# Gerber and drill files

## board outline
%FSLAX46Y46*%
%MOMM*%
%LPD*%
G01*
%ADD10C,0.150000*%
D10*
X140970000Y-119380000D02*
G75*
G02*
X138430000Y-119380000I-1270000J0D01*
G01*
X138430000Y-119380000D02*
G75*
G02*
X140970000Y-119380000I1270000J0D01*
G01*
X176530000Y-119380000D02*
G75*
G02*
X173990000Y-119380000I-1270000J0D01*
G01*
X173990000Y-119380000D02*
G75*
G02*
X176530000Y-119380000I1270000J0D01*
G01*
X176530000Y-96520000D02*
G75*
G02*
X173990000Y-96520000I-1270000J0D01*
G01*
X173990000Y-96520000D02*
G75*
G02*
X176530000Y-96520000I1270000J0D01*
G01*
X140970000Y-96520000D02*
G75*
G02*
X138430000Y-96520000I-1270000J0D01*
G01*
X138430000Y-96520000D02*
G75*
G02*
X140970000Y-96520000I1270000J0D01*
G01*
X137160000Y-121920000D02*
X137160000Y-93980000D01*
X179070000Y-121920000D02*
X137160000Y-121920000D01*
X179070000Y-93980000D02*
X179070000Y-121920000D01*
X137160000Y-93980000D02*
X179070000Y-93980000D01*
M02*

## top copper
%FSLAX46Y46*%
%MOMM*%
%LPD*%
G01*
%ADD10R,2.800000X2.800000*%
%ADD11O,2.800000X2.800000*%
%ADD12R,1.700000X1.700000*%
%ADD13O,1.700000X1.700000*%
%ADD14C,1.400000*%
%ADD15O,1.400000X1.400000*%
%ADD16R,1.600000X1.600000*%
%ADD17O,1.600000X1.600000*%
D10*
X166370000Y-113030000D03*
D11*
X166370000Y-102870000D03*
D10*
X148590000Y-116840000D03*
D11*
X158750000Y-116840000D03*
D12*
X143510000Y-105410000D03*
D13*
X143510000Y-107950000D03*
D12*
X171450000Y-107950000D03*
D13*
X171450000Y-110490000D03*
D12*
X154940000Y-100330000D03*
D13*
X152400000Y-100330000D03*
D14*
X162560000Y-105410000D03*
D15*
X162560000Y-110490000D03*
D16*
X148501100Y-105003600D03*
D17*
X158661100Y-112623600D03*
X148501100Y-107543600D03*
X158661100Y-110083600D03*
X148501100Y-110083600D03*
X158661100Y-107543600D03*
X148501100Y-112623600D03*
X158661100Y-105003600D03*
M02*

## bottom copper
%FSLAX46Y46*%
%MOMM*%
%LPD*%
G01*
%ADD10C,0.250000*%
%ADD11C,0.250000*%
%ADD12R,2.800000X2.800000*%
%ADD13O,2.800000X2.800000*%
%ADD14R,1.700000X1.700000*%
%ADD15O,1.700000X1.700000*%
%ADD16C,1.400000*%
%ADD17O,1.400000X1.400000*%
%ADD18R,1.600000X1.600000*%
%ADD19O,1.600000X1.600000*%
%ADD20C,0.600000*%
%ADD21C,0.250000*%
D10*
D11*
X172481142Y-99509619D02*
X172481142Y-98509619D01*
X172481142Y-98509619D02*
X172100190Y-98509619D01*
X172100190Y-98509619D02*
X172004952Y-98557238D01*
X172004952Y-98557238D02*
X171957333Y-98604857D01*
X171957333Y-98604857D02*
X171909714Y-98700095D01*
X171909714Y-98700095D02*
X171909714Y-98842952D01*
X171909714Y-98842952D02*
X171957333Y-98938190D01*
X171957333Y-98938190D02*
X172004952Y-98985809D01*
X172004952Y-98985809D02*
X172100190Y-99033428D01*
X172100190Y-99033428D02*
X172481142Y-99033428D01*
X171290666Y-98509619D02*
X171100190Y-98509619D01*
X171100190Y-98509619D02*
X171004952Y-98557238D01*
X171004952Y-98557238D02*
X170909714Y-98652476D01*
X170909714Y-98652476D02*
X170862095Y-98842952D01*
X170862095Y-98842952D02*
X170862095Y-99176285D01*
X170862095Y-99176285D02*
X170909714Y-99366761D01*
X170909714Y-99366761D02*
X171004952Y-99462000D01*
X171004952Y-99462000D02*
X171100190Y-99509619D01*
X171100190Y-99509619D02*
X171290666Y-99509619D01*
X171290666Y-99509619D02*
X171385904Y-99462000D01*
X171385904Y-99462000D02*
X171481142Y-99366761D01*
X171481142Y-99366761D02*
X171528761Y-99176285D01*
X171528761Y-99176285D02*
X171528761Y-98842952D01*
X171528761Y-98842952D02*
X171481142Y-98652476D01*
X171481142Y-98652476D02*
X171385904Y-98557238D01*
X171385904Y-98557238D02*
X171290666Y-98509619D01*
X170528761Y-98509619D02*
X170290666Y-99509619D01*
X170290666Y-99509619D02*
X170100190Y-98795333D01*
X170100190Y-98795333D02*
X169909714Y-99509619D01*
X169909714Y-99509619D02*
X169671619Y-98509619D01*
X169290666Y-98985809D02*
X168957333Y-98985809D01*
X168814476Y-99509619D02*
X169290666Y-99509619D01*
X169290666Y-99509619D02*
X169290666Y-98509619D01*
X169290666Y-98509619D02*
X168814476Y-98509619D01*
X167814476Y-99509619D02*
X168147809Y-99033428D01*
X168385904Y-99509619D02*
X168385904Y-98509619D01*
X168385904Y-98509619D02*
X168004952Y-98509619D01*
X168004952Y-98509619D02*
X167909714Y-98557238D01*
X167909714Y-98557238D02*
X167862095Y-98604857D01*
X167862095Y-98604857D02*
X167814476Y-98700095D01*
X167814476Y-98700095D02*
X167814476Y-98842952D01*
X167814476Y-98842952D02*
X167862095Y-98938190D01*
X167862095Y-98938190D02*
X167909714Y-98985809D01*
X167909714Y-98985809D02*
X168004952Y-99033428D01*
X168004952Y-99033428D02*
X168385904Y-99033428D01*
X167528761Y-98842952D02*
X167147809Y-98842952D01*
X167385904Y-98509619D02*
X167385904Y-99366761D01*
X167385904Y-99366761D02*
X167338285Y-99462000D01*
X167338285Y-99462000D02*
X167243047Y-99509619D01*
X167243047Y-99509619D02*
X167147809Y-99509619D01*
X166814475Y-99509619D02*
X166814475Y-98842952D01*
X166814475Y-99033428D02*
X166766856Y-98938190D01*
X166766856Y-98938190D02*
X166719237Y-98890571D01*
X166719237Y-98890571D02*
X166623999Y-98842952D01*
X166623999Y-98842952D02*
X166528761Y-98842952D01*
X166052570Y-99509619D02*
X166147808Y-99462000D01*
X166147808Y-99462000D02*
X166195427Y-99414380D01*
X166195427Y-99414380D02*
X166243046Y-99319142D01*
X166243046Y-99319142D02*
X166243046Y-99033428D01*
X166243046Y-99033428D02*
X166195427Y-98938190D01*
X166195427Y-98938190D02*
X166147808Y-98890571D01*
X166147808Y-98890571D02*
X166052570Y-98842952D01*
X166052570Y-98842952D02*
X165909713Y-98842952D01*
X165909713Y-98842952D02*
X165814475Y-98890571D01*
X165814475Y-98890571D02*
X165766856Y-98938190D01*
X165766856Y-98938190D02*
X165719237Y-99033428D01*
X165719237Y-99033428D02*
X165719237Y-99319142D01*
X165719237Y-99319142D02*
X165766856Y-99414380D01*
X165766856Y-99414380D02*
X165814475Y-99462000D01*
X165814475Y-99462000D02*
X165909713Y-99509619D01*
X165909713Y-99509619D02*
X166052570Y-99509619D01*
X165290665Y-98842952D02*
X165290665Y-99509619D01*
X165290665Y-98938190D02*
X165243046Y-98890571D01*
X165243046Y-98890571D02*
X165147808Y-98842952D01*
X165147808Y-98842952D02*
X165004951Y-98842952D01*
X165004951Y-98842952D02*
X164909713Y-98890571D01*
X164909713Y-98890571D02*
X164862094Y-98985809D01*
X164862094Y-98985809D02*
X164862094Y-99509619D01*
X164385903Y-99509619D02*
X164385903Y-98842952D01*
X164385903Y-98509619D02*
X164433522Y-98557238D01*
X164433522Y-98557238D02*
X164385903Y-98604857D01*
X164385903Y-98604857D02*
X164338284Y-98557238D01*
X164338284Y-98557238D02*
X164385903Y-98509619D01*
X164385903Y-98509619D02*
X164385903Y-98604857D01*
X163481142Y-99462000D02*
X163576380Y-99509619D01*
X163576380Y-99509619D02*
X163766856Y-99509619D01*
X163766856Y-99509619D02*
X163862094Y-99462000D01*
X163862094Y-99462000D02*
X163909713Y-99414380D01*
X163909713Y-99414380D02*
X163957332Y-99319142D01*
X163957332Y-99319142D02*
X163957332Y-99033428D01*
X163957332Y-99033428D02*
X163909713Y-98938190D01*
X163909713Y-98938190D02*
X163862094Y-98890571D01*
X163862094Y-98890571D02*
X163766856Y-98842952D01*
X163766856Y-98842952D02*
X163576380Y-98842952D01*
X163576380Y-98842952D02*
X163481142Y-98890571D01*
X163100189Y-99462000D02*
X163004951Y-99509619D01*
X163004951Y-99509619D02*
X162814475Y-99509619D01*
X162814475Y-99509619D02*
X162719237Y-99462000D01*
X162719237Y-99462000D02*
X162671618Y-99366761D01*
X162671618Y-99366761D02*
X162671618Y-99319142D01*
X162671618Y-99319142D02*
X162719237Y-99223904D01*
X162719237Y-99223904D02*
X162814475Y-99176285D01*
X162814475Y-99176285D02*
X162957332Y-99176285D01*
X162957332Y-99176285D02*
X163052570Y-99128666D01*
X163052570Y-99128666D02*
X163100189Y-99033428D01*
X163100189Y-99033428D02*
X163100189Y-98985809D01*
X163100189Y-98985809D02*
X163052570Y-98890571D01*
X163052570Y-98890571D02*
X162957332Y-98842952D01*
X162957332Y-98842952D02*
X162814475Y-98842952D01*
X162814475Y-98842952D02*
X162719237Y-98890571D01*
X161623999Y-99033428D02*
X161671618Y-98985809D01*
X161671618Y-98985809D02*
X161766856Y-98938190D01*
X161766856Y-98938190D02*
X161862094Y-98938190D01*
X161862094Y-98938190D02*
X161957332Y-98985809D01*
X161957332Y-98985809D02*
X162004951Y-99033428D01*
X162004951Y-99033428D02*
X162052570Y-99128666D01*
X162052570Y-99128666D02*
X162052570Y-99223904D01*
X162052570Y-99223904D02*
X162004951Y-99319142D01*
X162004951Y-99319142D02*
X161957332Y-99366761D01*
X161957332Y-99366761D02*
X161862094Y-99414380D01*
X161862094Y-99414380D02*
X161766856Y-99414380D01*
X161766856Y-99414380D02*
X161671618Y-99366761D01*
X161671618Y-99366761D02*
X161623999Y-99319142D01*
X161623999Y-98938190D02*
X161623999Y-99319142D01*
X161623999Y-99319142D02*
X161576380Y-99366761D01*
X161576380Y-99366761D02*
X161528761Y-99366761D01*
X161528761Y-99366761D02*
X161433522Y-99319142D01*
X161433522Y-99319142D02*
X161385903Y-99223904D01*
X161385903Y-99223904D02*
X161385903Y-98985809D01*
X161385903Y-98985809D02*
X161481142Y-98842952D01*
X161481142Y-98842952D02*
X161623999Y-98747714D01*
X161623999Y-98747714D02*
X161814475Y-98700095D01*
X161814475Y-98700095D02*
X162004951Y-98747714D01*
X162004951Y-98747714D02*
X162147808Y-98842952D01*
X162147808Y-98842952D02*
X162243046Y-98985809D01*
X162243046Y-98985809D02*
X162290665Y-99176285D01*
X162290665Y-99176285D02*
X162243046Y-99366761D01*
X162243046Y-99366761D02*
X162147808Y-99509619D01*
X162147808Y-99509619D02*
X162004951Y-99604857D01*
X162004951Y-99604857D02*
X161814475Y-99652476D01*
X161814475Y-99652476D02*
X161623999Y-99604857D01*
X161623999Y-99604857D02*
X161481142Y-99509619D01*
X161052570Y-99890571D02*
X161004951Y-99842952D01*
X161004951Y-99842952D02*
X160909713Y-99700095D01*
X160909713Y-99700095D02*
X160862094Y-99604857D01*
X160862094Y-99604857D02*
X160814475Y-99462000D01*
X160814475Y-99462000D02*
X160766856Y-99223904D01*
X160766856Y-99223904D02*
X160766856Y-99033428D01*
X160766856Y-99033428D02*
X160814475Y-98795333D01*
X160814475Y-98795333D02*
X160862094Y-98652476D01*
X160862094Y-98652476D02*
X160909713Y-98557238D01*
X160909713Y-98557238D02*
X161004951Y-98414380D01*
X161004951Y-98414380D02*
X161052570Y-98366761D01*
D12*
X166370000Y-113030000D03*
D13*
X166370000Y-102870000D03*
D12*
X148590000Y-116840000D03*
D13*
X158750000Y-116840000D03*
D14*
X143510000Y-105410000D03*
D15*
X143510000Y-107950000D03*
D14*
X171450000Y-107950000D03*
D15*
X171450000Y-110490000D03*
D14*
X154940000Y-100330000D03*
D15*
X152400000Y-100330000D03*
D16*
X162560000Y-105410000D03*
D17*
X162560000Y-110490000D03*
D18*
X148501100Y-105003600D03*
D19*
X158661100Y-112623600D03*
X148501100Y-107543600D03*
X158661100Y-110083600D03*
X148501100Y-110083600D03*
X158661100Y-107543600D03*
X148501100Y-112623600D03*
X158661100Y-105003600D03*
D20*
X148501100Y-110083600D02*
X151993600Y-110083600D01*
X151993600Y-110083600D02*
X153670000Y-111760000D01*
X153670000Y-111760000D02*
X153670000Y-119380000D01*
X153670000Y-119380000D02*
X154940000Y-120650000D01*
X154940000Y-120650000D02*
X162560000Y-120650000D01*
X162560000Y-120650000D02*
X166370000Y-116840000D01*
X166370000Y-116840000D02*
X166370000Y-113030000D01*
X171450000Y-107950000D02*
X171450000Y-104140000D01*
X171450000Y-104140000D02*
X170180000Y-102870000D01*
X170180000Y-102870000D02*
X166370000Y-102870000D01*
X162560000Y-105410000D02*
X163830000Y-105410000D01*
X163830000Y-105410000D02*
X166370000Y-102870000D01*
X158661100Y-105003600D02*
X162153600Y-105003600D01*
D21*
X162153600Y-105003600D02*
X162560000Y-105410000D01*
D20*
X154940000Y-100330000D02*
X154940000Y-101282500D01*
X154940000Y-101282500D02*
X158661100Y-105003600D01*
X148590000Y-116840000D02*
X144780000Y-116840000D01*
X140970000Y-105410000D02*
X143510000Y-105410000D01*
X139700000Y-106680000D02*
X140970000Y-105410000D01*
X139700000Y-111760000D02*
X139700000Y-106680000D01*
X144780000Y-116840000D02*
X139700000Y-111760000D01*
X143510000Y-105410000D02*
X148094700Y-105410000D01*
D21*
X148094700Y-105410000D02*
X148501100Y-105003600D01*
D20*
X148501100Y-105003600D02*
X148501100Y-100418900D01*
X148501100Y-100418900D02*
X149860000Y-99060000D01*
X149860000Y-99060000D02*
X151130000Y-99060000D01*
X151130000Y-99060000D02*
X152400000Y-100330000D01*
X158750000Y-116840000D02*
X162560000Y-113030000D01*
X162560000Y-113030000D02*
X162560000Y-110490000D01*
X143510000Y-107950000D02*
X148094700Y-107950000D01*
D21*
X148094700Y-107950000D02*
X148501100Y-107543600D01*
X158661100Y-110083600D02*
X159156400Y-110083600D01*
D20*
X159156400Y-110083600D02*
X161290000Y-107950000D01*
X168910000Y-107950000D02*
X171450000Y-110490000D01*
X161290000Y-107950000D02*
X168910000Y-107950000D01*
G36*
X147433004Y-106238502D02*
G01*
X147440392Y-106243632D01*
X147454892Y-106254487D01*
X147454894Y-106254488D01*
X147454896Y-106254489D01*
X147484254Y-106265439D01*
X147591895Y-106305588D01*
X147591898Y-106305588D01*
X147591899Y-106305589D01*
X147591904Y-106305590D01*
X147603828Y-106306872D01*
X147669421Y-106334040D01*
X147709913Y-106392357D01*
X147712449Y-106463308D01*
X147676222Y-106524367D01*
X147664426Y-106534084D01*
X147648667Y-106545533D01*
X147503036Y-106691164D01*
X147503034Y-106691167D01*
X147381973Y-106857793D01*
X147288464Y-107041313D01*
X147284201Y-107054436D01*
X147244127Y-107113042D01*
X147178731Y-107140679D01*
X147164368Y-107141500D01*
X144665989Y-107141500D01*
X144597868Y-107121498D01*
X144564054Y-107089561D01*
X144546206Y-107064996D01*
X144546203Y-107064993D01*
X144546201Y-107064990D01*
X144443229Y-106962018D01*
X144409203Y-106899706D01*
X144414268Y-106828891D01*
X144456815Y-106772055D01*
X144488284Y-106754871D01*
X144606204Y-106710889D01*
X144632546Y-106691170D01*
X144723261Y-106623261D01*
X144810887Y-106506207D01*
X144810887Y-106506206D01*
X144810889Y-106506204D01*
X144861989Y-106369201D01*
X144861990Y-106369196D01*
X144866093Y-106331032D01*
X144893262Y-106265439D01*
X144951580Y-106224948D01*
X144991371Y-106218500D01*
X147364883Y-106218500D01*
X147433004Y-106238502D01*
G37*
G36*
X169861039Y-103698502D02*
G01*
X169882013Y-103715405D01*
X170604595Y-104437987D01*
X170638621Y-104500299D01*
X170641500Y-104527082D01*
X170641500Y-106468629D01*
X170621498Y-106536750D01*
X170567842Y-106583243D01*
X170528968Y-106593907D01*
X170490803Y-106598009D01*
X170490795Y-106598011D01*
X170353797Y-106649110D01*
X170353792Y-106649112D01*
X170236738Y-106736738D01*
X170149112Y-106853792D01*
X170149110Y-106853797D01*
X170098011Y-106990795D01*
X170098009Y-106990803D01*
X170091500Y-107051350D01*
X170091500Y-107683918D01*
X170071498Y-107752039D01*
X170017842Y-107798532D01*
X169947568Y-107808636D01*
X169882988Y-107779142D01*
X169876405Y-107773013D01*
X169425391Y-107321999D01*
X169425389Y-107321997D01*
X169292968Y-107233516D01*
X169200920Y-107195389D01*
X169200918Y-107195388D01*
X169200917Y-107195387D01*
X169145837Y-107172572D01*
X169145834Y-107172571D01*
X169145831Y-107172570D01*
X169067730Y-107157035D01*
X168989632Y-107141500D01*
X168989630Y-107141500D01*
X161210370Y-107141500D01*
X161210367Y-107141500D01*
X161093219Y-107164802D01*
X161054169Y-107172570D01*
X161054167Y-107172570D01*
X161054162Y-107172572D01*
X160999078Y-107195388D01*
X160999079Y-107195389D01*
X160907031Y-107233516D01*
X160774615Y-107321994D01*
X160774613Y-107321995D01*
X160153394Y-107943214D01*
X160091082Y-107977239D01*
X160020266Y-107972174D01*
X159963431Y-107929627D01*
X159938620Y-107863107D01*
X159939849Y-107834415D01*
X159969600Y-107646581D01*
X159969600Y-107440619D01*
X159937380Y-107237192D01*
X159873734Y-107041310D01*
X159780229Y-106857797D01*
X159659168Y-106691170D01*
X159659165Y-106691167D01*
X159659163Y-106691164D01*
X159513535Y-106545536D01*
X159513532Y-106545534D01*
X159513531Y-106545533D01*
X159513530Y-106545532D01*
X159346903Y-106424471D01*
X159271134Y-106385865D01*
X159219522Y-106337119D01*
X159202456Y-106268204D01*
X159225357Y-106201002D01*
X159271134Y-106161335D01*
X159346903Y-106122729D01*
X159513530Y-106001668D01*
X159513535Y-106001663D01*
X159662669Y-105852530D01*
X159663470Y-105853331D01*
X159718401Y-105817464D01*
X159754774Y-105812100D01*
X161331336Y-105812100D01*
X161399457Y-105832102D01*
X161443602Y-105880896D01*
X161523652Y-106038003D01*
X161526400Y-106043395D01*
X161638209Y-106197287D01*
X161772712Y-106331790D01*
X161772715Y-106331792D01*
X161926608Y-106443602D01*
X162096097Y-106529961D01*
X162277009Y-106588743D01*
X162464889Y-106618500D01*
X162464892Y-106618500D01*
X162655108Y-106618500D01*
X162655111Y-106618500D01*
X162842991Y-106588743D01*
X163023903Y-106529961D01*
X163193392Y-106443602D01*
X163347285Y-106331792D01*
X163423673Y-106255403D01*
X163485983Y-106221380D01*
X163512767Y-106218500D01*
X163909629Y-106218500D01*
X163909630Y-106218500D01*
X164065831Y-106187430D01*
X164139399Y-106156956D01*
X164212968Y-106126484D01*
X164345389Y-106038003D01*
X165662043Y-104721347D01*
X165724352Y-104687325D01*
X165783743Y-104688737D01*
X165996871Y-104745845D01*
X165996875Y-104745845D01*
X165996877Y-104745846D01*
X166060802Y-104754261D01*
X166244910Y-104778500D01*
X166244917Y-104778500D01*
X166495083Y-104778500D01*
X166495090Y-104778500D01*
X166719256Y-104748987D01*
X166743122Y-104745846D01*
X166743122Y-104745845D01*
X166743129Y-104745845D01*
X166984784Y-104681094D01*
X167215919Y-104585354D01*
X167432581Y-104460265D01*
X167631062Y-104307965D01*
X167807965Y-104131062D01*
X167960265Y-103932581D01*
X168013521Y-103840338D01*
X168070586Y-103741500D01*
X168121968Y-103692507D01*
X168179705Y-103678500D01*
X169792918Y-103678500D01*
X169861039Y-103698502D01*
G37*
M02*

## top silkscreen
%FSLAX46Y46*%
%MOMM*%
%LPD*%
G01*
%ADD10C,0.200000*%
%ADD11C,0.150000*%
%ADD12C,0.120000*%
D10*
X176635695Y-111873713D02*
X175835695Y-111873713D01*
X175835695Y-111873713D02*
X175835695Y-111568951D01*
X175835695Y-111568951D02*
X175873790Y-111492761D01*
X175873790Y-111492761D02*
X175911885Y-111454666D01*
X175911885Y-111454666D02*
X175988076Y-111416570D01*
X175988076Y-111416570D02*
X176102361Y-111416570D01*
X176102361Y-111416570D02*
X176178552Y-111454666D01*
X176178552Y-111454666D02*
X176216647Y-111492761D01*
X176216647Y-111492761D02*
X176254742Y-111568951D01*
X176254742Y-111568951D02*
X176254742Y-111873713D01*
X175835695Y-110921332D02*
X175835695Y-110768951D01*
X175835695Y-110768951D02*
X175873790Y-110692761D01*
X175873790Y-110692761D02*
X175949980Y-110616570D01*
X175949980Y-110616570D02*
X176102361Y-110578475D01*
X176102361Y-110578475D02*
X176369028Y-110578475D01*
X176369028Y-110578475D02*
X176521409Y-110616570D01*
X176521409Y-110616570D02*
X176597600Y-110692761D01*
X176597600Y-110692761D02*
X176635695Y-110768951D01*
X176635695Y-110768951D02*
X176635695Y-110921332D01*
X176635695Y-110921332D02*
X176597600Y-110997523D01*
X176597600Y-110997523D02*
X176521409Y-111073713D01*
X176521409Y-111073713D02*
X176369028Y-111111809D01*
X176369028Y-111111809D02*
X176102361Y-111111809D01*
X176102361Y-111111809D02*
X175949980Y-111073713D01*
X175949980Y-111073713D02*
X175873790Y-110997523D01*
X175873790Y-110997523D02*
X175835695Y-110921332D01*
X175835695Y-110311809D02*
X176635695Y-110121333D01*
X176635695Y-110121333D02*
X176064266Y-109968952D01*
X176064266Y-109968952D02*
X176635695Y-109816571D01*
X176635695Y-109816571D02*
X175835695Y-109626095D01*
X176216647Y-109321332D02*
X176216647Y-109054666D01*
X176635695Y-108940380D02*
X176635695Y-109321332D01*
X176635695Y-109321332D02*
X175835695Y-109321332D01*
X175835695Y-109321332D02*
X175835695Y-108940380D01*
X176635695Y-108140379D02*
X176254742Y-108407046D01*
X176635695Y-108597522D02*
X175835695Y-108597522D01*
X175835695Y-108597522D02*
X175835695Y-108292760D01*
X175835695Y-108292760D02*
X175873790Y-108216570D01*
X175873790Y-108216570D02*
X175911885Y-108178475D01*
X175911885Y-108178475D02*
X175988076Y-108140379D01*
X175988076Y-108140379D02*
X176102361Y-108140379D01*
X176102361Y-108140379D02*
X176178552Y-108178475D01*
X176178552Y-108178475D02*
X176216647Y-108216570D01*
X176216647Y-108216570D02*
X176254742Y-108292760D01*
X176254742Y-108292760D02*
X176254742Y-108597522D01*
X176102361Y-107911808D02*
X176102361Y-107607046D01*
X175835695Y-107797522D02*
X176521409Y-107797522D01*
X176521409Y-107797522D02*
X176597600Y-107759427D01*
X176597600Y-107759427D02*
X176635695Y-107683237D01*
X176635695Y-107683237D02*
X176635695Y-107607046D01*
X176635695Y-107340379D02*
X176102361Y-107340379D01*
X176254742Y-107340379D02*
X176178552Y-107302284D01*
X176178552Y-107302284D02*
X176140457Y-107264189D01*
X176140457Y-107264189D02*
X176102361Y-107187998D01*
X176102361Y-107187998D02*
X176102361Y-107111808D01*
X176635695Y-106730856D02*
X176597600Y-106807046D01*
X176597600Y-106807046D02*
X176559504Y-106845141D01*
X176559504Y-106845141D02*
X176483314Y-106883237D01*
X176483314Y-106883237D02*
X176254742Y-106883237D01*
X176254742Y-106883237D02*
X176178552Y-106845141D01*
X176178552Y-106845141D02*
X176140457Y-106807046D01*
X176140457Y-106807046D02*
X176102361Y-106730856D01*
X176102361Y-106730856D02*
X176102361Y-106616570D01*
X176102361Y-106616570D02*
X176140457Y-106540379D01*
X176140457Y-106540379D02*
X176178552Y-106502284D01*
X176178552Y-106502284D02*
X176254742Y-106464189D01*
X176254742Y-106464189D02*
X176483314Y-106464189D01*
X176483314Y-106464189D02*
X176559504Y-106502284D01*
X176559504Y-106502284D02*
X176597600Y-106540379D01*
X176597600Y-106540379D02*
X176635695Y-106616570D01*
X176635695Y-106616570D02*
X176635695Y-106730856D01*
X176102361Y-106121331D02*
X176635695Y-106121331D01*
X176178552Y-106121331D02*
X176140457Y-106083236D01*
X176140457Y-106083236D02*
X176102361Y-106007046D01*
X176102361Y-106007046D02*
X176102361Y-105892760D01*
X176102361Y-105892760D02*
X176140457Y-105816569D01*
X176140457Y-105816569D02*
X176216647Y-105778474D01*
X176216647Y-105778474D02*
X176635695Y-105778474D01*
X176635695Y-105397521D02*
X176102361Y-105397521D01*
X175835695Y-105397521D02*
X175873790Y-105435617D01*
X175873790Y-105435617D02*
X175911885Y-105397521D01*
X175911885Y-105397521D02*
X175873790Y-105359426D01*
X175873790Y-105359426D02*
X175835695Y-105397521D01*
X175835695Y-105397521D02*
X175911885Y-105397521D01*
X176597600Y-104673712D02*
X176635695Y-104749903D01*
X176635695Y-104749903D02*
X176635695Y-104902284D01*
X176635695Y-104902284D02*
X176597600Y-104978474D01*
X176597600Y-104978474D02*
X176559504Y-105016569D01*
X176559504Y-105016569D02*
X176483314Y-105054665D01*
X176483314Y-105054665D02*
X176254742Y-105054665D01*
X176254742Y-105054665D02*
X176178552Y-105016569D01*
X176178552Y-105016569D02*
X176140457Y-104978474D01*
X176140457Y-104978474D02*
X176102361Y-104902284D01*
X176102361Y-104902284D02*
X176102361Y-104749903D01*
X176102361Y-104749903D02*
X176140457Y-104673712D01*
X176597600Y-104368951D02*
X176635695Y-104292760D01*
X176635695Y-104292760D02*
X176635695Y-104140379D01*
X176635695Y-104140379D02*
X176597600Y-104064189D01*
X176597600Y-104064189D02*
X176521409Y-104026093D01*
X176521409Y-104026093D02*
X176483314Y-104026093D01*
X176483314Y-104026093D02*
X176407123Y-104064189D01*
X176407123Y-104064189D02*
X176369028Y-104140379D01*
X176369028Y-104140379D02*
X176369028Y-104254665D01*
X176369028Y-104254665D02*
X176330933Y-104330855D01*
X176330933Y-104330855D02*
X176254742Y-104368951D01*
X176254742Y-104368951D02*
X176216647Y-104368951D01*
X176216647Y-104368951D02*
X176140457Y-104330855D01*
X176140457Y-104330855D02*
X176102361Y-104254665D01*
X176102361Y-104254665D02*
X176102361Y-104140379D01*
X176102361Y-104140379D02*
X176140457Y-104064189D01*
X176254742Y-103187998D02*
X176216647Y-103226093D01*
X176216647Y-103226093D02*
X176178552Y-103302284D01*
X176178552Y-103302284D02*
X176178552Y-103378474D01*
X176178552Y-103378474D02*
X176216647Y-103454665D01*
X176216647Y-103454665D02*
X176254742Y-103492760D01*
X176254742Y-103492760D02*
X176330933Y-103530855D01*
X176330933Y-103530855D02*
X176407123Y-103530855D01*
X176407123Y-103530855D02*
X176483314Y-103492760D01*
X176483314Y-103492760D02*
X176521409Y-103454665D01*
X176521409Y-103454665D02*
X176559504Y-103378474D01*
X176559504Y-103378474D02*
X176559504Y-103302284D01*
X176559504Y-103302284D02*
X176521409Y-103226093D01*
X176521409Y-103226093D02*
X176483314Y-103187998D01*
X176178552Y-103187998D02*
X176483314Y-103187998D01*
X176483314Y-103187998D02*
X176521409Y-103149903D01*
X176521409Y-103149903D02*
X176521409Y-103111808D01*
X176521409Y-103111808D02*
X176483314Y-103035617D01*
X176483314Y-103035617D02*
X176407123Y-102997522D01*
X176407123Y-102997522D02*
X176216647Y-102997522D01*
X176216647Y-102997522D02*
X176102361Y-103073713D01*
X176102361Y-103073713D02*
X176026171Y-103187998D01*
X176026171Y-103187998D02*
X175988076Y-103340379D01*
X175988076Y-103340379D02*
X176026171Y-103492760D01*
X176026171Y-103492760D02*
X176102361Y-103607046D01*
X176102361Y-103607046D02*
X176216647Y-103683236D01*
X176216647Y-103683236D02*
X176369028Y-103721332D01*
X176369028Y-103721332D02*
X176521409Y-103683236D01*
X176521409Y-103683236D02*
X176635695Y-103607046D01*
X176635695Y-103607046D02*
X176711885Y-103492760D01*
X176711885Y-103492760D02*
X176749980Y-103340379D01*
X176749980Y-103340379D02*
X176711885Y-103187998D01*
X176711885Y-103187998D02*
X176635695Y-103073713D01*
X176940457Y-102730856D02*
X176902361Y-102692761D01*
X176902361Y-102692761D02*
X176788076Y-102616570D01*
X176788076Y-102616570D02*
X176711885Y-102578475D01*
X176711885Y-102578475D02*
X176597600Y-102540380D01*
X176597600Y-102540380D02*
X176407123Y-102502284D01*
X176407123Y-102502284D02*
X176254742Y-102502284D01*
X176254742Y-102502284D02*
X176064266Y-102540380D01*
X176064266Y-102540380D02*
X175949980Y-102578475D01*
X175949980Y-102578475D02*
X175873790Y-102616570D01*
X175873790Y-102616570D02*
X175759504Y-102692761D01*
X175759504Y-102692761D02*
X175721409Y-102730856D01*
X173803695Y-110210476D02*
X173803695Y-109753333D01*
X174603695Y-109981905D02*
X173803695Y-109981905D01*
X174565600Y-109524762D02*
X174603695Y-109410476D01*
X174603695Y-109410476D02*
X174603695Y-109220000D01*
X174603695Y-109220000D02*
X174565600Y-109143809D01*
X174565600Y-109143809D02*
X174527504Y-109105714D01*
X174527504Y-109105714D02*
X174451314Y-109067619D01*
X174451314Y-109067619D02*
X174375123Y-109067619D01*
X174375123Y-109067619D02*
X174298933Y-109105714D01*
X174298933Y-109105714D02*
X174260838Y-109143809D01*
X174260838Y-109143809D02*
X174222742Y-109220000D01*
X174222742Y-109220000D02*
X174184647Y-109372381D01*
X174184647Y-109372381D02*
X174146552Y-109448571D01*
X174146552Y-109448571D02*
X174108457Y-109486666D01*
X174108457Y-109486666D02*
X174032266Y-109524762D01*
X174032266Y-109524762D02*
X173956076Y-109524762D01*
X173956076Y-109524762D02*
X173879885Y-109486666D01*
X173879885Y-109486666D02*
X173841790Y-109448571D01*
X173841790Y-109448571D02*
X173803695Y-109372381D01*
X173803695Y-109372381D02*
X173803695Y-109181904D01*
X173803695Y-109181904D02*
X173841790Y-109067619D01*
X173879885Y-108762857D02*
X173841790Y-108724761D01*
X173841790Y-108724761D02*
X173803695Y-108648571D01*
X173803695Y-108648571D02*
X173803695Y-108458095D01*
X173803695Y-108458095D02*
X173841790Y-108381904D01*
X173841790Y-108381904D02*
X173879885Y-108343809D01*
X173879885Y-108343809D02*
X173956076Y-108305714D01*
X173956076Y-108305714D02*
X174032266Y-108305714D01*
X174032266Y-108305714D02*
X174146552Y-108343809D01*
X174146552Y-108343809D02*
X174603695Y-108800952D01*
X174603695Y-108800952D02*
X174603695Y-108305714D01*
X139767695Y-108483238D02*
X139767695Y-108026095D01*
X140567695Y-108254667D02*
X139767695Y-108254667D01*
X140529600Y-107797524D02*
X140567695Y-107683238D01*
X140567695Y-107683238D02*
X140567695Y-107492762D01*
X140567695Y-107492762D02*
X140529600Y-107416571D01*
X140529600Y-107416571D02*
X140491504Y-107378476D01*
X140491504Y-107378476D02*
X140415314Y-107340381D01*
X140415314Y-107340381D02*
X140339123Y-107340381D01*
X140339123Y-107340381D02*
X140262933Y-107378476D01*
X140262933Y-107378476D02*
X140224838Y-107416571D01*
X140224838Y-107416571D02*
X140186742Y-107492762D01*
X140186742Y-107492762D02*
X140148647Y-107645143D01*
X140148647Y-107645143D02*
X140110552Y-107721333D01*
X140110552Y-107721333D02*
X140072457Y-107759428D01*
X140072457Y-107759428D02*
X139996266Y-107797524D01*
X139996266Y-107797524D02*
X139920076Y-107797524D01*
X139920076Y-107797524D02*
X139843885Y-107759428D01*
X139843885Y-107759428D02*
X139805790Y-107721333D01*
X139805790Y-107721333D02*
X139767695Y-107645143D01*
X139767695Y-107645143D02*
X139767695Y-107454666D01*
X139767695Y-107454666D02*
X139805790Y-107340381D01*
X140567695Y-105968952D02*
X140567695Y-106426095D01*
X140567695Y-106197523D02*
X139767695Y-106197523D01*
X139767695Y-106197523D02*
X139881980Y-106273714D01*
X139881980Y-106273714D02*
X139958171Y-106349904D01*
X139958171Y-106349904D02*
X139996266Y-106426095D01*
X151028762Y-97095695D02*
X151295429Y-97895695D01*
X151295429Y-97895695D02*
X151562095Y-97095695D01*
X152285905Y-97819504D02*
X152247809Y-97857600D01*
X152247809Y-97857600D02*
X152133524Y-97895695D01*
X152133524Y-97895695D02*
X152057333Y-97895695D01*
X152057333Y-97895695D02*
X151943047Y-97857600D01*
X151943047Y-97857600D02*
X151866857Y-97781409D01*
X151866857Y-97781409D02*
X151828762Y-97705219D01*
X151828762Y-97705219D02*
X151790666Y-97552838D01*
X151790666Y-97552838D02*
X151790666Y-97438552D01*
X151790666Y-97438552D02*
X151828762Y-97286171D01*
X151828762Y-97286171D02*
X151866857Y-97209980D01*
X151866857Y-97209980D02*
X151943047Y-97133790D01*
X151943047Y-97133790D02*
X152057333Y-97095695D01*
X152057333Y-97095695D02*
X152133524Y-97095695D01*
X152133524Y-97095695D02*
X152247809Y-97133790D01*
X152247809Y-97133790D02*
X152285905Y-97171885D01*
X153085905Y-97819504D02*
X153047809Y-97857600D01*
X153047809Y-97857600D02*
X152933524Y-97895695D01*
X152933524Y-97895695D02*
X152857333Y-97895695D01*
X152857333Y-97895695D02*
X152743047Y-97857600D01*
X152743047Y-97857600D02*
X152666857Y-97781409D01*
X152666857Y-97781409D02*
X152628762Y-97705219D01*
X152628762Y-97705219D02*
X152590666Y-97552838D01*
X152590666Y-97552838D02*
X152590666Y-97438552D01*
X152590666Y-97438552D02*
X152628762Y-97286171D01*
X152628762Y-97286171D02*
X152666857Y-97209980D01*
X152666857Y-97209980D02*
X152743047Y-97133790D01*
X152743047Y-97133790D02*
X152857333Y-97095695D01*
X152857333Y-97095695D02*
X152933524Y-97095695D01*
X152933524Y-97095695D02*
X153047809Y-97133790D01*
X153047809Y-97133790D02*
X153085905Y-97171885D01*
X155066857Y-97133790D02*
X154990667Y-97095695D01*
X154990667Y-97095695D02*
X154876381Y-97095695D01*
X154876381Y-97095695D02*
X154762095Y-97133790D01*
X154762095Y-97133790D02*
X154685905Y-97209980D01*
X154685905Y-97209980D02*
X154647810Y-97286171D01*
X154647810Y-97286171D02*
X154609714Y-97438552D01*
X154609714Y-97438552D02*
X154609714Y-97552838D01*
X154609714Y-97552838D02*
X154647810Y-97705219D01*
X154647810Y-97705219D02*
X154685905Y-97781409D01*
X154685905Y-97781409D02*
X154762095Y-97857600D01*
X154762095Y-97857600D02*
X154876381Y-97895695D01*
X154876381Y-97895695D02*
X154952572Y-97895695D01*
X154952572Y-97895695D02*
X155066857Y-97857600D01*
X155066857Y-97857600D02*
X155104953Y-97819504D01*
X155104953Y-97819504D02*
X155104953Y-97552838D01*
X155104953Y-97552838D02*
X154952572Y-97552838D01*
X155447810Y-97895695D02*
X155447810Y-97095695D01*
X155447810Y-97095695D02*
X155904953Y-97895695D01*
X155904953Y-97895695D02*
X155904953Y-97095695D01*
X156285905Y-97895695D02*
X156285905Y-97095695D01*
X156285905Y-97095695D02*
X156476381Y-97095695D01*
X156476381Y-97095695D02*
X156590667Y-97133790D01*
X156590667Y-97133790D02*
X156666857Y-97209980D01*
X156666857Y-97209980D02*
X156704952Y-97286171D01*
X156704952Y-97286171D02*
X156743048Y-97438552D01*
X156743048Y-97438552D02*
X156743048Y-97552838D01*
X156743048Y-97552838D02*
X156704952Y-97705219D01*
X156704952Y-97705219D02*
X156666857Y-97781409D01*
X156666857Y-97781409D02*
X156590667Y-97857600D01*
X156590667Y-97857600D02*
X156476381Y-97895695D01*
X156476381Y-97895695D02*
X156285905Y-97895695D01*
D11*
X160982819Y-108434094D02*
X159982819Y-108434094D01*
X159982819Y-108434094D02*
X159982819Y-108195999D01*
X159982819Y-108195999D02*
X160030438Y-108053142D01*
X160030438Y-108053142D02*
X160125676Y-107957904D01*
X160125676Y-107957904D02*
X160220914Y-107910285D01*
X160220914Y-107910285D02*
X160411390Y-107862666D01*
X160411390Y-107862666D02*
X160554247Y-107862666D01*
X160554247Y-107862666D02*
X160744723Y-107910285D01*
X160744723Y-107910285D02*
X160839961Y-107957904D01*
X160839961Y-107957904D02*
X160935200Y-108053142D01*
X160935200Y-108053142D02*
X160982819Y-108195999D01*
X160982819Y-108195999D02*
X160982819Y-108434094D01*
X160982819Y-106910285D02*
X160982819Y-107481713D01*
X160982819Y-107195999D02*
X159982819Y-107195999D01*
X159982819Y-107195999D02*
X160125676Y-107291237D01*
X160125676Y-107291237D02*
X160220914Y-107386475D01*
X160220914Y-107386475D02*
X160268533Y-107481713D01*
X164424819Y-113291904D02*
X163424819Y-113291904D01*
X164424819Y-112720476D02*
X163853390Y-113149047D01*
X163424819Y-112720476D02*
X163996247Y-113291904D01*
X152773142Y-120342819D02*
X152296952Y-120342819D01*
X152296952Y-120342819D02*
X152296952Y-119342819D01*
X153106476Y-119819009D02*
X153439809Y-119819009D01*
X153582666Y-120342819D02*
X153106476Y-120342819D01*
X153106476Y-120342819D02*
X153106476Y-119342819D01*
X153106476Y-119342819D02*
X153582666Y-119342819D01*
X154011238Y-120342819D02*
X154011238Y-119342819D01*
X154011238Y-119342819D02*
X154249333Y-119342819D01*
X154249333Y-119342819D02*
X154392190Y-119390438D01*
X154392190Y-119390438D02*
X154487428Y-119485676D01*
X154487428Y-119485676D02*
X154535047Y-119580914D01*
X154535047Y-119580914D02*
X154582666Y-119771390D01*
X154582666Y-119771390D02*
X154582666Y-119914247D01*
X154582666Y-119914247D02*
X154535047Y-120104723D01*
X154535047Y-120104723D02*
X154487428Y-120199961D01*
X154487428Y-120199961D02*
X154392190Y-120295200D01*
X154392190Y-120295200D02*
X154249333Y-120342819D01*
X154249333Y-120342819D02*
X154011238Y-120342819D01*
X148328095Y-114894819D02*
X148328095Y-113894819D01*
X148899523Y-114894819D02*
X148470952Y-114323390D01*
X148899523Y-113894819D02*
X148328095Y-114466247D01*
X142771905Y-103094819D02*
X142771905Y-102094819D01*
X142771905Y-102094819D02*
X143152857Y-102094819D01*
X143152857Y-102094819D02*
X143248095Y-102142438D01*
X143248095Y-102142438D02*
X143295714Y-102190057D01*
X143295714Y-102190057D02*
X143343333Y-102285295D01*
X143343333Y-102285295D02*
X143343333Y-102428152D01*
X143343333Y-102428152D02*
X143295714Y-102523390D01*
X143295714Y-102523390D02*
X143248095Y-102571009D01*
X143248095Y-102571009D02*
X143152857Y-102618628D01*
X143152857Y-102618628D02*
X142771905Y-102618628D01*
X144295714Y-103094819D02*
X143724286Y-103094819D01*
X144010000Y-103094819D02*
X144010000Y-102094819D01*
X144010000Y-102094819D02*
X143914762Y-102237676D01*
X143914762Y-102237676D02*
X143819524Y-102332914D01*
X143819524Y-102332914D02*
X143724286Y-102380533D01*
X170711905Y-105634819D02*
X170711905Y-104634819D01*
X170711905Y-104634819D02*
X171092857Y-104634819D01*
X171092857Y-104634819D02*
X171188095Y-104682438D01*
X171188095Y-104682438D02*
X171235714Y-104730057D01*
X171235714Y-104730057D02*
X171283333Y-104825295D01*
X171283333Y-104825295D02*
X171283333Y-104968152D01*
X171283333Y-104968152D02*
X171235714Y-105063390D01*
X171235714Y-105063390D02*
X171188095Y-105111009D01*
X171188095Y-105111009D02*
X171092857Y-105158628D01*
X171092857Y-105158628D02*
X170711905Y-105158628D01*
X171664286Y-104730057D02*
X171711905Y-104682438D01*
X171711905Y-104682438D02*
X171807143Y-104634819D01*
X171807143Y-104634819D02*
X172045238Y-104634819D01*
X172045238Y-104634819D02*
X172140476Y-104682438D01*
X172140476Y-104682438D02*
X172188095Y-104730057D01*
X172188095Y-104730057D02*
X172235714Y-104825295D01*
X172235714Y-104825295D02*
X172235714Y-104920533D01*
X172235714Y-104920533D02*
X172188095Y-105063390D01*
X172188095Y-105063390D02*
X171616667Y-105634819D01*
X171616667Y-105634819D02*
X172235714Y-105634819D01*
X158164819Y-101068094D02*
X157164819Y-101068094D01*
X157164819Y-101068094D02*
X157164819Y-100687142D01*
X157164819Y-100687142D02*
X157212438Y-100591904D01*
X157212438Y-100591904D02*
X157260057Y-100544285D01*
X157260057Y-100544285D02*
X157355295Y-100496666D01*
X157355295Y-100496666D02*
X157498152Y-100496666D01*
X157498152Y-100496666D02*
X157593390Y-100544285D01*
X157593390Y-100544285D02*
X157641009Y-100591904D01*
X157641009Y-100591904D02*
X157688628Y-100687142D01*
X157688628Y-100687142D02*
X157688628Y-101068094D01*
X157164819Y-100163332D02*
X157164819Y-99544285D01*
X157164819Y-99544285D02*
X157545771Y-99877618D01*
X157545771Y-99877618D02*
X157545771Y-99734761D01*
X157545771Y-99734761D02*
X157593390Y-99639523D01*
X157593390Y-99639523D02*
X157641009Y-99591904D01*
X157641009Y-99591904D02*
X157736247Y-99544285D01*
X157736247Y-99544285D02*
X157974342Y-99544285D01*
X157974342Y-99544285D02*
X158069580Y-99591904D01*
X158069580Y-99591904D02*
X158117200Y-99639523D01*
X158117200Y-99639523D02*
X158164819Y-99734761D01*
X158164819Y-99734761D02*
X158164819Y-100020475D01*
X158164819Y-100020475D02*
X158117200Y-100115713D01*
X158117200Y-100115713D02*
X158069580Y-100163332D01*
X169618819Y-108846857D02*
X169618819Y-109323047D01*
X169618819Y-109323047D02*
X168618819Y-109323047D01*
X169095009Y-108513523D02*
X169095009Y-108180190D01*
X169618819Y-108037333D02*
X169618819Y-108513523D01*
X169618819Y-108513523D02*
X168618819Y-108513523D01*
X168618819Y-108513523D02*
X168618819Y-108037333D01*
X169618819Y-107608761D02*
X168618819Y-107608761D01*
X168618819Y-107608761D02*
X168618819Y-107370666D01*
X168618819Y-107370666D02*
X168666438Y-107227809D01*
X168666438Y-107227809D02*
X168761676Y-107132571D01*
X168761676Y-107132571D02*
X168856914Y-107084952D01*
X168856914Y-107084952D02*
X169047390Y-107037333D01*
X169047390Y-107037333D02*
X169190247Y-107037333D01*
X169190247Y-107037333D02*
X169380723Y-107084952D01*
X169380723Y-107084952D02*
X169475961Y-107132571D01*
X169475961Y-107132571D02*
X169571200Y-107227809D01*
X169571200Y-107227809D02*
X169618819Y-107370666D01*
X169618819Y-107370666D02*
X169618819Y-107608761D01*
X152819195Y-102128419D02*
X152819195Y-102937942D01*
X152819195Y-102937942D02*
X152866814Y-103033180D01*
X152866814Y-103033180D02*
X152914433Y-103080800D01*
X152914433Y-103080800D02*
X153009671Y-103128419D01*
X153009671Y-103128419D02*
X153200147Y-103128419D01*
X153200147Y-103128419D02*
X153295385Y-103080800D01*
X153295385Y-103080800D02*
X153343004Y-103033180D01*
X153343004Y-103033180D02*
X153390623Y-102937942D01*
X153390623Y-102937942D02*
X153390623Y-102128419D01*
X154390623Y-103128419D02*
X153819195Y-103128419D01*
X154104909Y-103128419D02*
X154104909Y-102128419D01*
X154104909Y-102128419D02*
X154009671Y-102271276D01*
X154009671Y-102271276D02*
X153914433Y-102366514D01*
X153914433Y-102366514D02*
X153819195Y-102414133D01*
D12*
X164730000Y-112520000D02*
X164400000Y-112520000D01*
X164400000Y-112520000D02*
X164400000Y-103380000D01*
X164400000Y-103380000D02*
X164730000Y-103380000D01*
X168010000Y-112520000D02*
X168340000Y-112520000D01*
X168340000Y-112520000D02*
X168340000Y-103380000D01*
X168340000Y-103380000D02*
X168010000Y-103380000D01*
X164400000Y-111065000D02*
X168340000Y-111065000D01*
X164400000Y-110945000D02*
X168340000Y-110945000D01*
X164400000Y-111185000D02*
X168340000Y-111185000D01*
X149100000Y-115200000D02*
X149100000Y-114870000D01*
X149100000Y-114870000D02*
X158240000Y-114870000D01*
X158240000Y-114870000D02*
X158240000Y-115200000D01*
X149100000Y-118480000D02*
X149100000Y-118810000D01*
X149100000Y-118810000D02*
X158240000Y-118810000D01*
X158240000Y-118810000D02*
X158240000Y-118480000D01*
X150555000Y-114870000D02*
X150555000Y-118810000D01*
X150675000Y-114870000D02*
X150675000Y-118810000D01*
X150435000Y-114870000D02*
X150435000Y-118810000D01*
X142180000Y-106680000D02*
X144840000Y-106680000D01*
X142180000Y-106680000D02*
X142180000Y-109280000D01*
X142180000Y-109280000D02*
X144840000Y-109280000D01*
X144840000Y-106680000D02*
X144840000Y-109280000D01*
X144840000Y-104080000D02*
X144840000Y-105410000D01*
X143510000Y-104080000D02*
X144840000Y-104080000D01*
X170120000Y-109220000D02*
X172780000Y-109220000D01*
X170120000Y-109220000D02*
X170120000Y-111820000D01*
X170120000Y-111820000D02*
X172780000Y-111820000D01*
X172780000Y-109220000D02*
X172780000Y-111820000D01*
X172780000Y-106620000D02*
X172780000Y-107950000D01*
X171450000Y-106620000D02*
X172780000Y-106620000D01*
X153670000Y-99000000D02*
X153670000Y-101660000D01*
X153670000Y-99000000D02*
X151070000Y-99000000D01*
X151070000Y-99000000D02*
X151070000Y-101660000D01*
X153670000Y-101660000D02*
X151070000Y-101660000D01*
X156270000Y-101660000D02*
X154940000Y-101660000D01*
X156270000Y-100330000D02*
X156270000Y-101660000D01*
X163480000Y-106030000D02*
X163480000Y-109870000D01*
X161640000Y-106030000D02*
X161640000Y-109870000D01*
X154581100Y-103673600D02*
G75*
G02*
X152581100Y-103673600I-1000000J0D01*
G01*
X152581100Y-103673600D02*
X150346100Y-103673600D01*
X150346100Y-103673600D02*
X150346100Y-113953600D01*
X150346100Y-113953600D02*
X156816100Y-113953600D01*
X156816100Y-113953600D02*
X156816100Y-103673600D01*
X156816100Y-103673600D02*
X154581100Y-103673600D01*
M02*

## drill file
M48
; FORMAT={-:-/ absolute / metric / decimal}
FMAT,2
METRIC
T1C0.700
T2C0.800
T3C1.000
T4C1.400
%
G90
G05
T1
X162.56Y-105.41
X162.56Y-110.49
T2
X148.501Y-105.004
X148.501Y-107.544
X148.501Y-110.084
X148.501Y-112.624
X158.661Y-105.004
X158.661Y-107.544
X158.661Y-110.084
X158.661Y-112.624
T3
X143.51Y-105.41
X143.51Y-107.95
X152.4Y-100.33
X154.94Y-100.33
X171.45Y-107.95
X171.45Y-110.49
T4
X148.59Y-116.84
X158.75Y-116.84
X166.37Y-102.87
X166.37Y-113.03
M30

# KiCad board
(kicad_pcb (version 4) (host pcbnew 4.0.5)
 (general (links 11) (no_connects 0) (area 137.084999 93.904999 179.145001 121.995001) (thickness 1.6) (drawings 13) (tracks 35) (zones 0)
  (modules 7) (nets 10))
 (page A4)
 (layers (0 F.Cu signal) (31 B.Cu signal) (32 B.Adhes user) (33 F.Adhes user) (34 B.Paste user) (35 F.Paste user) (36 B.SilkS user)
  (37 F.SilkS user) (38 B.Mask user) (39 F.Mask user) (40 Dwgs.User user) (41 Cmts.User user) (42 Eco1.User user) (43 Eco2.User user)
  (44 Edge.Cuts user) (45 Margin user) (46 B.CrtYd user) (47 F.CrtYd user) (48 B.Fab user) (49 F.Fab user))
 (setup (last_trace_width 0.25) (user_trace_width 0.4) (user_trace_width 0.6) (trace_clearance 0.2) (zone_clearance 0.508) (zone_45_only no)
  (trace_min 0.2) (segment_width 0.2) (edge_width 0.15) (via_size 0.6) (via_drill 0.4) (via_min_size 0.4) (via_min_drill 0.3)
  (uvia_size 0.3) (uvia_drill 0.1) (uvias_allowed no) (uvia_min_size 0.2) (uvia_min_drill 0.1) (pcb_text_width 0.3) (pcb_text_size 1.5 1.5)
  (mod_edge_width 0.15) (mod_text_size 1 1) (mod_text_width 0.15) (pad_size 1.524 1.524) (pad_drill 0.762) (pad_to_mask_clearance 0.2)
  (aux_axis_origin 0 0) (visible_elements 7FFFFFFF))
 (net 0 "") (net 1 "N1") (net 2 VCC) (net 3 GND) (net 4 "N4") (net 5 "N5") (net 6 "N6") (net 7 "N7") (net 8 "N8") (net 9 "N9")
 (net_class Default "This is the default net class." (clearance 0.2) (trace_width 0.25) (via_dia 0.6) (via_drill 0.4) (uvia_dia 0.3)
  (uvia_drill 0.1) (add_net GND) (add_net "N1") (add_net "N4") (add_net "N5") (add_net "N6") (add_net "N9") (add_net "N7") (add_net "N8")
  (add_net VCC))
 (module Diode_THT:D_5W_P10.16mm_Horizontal (layer F.Cu) (at 166.37 113.03 90)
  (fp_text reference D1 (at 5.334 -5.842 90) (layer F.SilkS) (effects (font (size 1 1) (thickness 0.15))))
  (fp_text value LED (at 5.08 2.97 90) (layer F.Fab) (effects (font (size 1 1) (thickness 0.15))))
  (fp_line (start 0.51 -1.64) (end 0.51 -1.97) (layer F.SilkS) (width 0.12))
  (fp_line (start 0.51 -1.97) (end 9.65 -1.97) (layer F.SilkS) (width 0.12))
  (fp_line (start 9.65 -1.97) (end 9.65 -1.64) (layer F.SilkS) (width 0.12))
  (fp_line (start 0.51 1.64) (end 0.51 1.97) (layer F.SilkS) (width 0.12))
  (fp_line (start 0.51 1.97) (end 9.65 1.97) (layer F.SilkS) (width 0.12))
  (fp_line (start 9.65 1.97) (end 9.65 1.64) (layer F.SilkS) (width 0.12))
  (fp_line (start 1.965 -1.97) (end 1.965 1.97) (layer F.SilkS) (width 0.12))
  (fp_line (start 2.085 -1.97) (end 2.085 1.97) (layer F.SilkS) (width 0.12))
  (fp_line (start 1.845 -1.97) (end 1.845 1.97) (layer F.SilkS) (width 0.12))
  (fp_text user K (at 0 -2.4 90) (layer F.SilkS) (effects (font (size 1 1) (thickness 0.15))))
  (pad 1 thru_hole rect (at 0 0 90) (size 2.8 2.8) (drill 1.4) (layers *.Cu *.Mask) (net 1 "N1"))
  (pad 2 thru_hole oval (at 10.16 0 90) (size 2.8 2.8) (drill 1.4) (layers *.Cu *.Mask) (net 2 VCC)))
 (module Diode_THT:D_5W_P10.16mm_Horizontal (layer F.Cu) (at 148.59 116.84)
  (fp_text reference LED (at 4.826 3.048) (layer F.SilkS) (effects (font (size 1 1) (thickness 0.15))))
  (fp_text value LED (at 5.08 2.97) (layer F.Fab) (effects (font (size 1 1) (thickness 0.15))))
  (fp_line (start 0.51 -1.64) (end 0.51 -1.97) (layer F.SilkS) (width 0.12))
  (fp_line (start 0.51 -1.97) (end 9.65 -1.97) (layer F.SilkS) (width 0.12))
  (fp_line (start 9.65 -1.97) (end 9.65 -1.64) (layer F.SilkS) (width 0.12))
  (fp_line (start 0.51 1.64) (end 0.51 1.97) (layer F.SilkS) (width 0.12))
  (fp_line (start 0.51 1.97) (end 9.65 1.97) (layer F.SilkS) (width 0.12))
  (fp_line (start 9.65 1.97) (end 9.65 1.64) (layer F.SilkS) (width 0.12))
  (fp_line (start 1.965 -1.97) (end 1.965 1.97) (layer F.SilkS) (width 0.12))
  (fp_line (start 2.085 -1.97) (end 2.085 1.97) (layer F.SilkS) (width 0.12))
  (fp_line (start 1.845 -1.97) (end 1.845 1.97) (layer F.SilkS) (width 0.12))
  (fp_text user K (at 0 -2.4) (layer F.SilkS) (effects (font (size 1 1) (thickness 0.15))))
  (pad 1 thru_hole rect (at 0 0) (size 2.8 2.8) (drill 1.4) (layers *.Cu *.Mask) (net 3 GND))
  (pad 2 thru_hole oval (at 10.16 0) (size 2.8 2.8) (drill 1.4) (layers *.Cu *.Mask) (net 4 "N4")))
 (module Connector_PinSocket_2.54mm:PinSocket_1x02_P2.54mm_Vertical (layer F.Cu) (at 143.51 105.41)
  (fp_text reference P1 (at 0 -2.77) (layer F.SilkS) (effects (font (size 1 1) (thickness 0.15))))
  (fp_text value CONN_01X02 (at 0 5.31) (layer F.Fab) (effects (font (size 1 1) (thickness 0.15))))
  (fp_line (start -1.33 1.27) (end 1.33 1.27) (layer F.SilkS) (width 0.12))
  (fp_line (start -1.33 1.27) (end -1.33 3.87) (layer F.SilkS) (width 0.12))
  (fp_line (start -1.33 3.87) (end 1.33 3.87) (layer F.SilkS) (width 0.12))
  (fp_line (start 1.33 1.27) (end 1.33 3.87) (layer F.SilkS) (width 0.12))
  (fp_line (start 1.33 -1.33) (end 1.33 0) (layer F.SilkS) (width 0.12))
  (fp_line (start 0 -1.33) (end 1.33 -1.33) (layer F.SilkS) (width 0.12))
  (pad 1 thru_hole rect (at 0 0) (size 1.7 1.7) (drill 1) (layers *.Cu *.Mask) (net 3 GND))
  (pad 2 thru_hole oval (at 0 2.54) (size 1.7 1.7) (drill 1) (layers *.Cu *.Mask) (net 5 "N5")))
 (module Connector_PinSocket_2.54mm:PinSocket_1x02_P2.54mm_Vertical (layer F.Cu) (at 171.45 107.95)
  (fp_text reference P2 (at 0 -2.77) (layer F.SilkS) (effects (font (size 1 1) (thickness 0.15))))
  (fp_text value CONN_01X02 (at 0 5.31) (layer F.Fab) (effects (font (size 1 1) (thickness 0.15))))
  (fp_line (start -1.33 1.27) (end 1.33 1.27) (layer F.SilkS) (width 0.12))
  (fp_line (start -1.33 1.27) (end -1.33 3.87) (layer F.SilkS) (width 0.12))
  (fp_line (start -1.33 3.87) (end 1.33 3.87) (layer F.SilkS) (width 0.12))
  (fp_line (start 1.33 1.27) (end 1.33 3.87) (layer F.SilkS) (width 0.12))
  (fp_line (start 1.33 -1.33) (end 1.33 0) (layer F.SilkS) (width 0.12))
  (fp_line (start 0 -1.33) (end 1.33 -1.33) (layer F.SilkS) (width 0.12))
  (pad 1 thru_hole rect (at 0 0) (size 1.7 1.7) (drill 1) (layers *.Cu *.Mask) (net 2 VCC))
  (pad 2 thru_hole oval (at 0 2.54) (size 1.7 1.7) (drill 1) (layers *.Cu *.Mask) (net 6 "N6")))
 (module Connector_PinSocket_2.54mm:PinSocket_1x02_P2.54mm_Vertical (layer F.Cu) (at 154.94 100.33 270)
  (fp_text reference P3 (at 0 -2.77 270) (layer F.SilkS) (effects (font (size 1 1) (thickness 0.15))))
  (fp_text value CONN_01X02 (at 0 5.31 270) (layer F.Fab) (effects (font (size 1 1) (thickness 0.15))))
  (fp_line (start -1.33 1.27) (end 1.33 1.27) (layer F.SilkS) (width 0.12))
  (fp_line (start -1.33 1.27) (end -1.33 3.87) (layer F.SilkS) (width 0.12))
  (fp_line (start -1.33 3.87) (end 1.33 3.87) (layer F.SilkS) (width 0.12))
  (fp_line (start 1.33 1.27) (end 1.33 3.87) (layer F.SilkS) (width 0.12))
  (fp_line (start 1.33 -1.33) (end 1.33 0) (layer F.SilkS) (width 0.12))
  (fp_line (start 0 -1.33) (end 1.33 -1.33) (layer F.SilkS) (width 0.12))
  (pad 1 thru_hole rect (at 0 0 270) (size 1.7 1.7) (drill 1) (layers *.Cu *.Mask) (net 2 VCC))
  (pad 2 thru_hole oval (at 0 2.54 270) (size 1.7 1.7) (drill 1) (layers *.Cu *.Mask) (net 3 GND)))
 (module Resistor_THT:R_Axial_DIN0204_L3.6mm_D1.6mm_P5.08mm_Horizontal (layer F.Cu) (at 162.56 105.41 270)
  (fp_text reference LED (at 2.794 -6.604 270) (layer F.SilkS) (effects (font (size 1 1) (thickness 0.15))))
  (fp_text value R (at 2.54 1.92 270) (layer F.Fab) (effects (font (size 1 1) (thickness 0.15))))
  (fp_line (start 0.62 -0.92) (end 4.46 -0.92) (layer F.SilkS) (width 0.12))
  (fp_line (start 0.62 0.92) (end 4.46 0.92) (layer F.SilkS) (width 0.12))
  (pad 1 thru_hole circle (at 0 0 270) (size 1.4 1.4) (drill 0.7) (layers *.Cu *.Mask) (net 2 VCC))
  (pad 2 thru_hole oval (at 5.08 0 270) (size 1.4 1.4) (drill 0.7) (layers *.Cu *.Mask) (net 4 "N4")))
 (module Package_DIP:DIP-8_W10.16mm (layer F.Cu) (at 148.5011 105.0036)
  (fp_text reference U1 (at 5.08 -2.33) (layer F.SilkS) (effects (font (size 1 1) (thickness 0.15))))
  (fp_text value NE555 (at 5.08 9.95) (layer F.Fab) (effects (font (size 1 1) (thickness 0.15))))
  (fp_arc (start 5.08 -1.33) (end 4.08 -1.33) (angle -180) (layer F.SilkS) (width 0.12))
  (fp_line (start 4.08 -1.33) (end 1.845 -1.33) (layer F.SilkS) (width 0.12))
  (fp_line (start 1.845 -1.33) (end 1.845 8.95) (layer F.SilkS) (width 0.12))
  (fp_line (start 1.845 8.95) (end 8.315 8.95) (layer F.SilkS) (width 0.12))
  (fp_line (start 8.315 8.95) (end 8.315 -1.33) (layer F.SilkS) (width 0.12))
  (fp_line (start 8.315 -1.33) (end 6.08 -1.33) (layer F.SilkS) (width 0.12))
  (pad 1 thru_hole rect (at 0 0) (size 1.6 1.6) (drill 0.8) (layers *.Cu *.Mask) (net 3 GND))
  (pad 5 thru_hole oval (at 10.16 7.62) (size 1.6 1.6) (drill 0.8) (layers *.Cu *.Mask) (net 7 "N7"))
  (pad 2 thru_hole oval (at 0 2.54) (size 1.6 1.6) (drill 0.8) (layers *.Cu *.Mask) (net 5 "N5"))
  (pad 6 thru_hole oval (at 10.16 5.08) (size 1.6 1.6) (drill 0.8) (layers *.Cu *.Mask) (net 6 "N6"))
  (pad 3 thru_hole oval (at 0 5.08) (size 1.6 1.6) (drill 0.8) (layers *.Cu *.Mask) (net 1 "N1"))
  (pad 7 thru_hole oval (at 10.16 2.54) (size 1.6 1.6) (drill 0.8) (layers *.Cu *.Mask) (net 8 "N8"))
  (pad 4 thru_hole oval (at 0 7.62) (size 1.6 1.6) (drill 0.8) (layers *.Cu *.Mask) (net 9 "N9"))
  (pad 8 thru_hole oval (at 10.16 0) (size 1.6 1.6) (drill 0.8) (layers *.Cu *.Mask) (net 2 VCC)))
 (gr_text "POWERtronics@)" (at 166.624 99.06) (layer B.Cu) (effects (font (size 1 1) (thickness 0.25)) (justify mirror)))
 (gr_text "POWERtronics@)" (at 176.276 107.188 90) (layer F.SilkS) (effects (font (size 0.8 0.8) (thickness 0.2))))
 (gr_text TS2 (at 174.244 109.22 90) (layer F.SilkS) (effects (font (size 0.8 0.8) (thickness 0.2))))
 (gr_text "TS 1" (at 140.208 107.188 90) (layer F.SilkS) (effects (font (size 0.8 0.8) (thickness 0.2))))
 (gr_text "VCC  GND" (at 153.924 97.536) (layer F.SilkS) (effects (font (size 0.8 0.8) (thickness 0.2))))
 (gr_circle (center 139.7 119.38) (end 139.7 118.11) (layer Edge.Cuts) (width 0.15))
 (gr_circle (center 175.26 119.38) (end 175.26 118.11) (layer Edge.Cuts) (width 0.15))
 (gr_circle (center 175.26 96.52) (end 176.53 96.52) (layer Edge.Cuts) (width 0.15))
 (gr_circle (center 139.7 96.52) (end 139.7 95.25) (layer Edge.Cuts) (width 0.15))
 (gr_line (start 137.16 121.92) (end 137.16 93.98) (angle 90) (layer Edge.Cuts) (width 0.15))
 (gr_line (start 179.07 121.92) (end 137.16 121.92) (angle 90) (layer Edge.Cuts) (width 0.15))
 (gr_line (start 179.07 93.98) (end 179.07 121.92) (angle 90) (layer Edge.Cuts) (width 0.15))
 (gr_line (start 137.16 93.98) (end 179.07 93.98) (angle 90) (layer Edge.Cuts) (width 0.15))
 (segment (start 148.5011 110.0836) (end 151.9936 110.0836) (width 0.6) (layer B.Cu) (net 1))
 (segment (start 151.9936 110.0836) (end 153.67 111.76) (width 0.6) (layer B.Cu) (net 1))
 (segment (start 153.67 111.76) (end 153.67 119.38) (width 0.6) (layer B.Cu) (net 1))
 (segment (start 153.67 119.38) (end 154.94 120.65) (width 0.6) (layer B.Cu) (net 1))
 (segment (start 154.94 120.65) (end 162.56 120.65) (width 0.6) (layer B.Cu) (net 1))
 (segment (start 162.56 120.65) (end 166.37 116.84) (width 0.6) (layer B.Cu) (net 1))
 (segment (start 166.37 116.84) (end 166.37 113.03) (width 0.6) (layer B.Cu) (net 1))
 (segment (start 171.45 107.95) (end 171.45 104.14) (width 0.6) (layer B.Cu) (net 2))
 (segment (start 171.45 104.14) (end 170.18 102.87) (width 0.6) (layer B.Cu) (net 2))
 (segment (start 170.18 102.87) (end 166.37 102.87) (width 0.6) (layer B.Cu) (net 2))
 (segment (start 162.56 105.41) (end 163.83 105.41) (width 0.6) (layer B.Cu) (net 2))
 (segment (start 163.83 105.41) (end 166.37 102.87) (width 0.6) (layer B.Cu) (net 2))
 (segment (start 158.6611 105.0036) (end 162.1536 105.0036) (width 0.6) (layer B.Cu) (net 2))
 (segment (start 162.1536 105.0036) (end 162.56 105.41) (width 0.25) (layer B.Cu) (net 2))
 (segment (start 154.94 100.33) (end 154.94 101.2825) (width 0.6) (layer B.Cu) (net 2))
 (segment (start 154.94 101.2825) (end 158.6611 105.0036) (width 0.6) (layer B.Cu) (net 2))
 (segment (start 148.59 116.84) (end 144.78 116.84) (width 0.6) (layer B.Cu) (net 3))
 (segment (start 140.97 105.41) (end 143.51 105.41) (width 0.6) (layer B.Cu) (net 3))
 (segment (start 139.7 106.68) (end 140.97 105.41) (width 0.6) (layer B.Cu) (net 3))
 (segment (start 139.7 111.76) (end 139.7 106.68) (width 0.6) (layer B.Cu) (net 3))
 (segment (start 144.78 116.84) (end 139.7 111.76) (width 0.6) (layer B.Cu) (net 3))
 (segment (start 143.51 105.41) (end 148.0947 105.41) (width 0.6) (layer B.Cu) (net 3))
 (segment (start 148.0947 105.41) (end 148.5011 105.0036) (width 0.25) (layer B.Cu) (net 3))
 (segment (start 148.5011 105.0036) (end 148.5011 100.4189) (width 0.6) (layer B.Cu) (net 3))
 (segment (start 148.5011 100.4189) (end 149.86 99.06) (width 0.6) (layer B.Cu) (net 3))
 (segment (start 149.86 99.06) (end 151.13 99.06) (width 0.6) (layer B.Cu) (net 3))
 (segment (start 151.13 99.06) (end 152.4 100.33) (width 0.6) (layer B.Cu) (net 3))
 (segment (start 158.75 116.84) (end 162.56 113.03) (width 0.6) (layer B.Cu) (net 4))
 (segment (start 162.56 113.03) (end 162.56 110.49) (width 0.6) (layer B.Cu) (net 4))
 (segment (start 143.51 107.95) (end 148.0947 107.95) (width 0.6) (layer B.Cu) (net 5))
 (segment (start 148.0947 107.95) (end 148.5011 107.5436) (width 0.25) (layer B.Cu) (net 5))
 (segment (start 158.6611 110.0836) (end 159.1564 110.0836) (width 0.25) (layer B.Cu) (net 6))
 (segment (start 159.1564 110.0836) (end 161.29 107.95) (width 0.6) (layer B.Cu) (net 6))
 (segment (start 168.91 107.95) (end 171.45 110.49) (width 0.6) (layer B.Cu) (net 6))
 (segment (start 161.29 107.95) (end 168.91 107.95) (width 0.6) (layer B.Cu) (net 6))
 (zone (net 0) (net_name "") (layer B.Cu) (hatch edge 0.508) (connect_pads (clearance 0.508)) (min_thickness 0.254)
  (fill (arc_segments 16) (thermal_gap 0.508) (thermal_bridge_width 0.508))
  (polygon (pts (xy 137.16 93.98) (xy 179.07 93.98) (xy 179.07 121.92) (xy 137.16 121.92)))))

